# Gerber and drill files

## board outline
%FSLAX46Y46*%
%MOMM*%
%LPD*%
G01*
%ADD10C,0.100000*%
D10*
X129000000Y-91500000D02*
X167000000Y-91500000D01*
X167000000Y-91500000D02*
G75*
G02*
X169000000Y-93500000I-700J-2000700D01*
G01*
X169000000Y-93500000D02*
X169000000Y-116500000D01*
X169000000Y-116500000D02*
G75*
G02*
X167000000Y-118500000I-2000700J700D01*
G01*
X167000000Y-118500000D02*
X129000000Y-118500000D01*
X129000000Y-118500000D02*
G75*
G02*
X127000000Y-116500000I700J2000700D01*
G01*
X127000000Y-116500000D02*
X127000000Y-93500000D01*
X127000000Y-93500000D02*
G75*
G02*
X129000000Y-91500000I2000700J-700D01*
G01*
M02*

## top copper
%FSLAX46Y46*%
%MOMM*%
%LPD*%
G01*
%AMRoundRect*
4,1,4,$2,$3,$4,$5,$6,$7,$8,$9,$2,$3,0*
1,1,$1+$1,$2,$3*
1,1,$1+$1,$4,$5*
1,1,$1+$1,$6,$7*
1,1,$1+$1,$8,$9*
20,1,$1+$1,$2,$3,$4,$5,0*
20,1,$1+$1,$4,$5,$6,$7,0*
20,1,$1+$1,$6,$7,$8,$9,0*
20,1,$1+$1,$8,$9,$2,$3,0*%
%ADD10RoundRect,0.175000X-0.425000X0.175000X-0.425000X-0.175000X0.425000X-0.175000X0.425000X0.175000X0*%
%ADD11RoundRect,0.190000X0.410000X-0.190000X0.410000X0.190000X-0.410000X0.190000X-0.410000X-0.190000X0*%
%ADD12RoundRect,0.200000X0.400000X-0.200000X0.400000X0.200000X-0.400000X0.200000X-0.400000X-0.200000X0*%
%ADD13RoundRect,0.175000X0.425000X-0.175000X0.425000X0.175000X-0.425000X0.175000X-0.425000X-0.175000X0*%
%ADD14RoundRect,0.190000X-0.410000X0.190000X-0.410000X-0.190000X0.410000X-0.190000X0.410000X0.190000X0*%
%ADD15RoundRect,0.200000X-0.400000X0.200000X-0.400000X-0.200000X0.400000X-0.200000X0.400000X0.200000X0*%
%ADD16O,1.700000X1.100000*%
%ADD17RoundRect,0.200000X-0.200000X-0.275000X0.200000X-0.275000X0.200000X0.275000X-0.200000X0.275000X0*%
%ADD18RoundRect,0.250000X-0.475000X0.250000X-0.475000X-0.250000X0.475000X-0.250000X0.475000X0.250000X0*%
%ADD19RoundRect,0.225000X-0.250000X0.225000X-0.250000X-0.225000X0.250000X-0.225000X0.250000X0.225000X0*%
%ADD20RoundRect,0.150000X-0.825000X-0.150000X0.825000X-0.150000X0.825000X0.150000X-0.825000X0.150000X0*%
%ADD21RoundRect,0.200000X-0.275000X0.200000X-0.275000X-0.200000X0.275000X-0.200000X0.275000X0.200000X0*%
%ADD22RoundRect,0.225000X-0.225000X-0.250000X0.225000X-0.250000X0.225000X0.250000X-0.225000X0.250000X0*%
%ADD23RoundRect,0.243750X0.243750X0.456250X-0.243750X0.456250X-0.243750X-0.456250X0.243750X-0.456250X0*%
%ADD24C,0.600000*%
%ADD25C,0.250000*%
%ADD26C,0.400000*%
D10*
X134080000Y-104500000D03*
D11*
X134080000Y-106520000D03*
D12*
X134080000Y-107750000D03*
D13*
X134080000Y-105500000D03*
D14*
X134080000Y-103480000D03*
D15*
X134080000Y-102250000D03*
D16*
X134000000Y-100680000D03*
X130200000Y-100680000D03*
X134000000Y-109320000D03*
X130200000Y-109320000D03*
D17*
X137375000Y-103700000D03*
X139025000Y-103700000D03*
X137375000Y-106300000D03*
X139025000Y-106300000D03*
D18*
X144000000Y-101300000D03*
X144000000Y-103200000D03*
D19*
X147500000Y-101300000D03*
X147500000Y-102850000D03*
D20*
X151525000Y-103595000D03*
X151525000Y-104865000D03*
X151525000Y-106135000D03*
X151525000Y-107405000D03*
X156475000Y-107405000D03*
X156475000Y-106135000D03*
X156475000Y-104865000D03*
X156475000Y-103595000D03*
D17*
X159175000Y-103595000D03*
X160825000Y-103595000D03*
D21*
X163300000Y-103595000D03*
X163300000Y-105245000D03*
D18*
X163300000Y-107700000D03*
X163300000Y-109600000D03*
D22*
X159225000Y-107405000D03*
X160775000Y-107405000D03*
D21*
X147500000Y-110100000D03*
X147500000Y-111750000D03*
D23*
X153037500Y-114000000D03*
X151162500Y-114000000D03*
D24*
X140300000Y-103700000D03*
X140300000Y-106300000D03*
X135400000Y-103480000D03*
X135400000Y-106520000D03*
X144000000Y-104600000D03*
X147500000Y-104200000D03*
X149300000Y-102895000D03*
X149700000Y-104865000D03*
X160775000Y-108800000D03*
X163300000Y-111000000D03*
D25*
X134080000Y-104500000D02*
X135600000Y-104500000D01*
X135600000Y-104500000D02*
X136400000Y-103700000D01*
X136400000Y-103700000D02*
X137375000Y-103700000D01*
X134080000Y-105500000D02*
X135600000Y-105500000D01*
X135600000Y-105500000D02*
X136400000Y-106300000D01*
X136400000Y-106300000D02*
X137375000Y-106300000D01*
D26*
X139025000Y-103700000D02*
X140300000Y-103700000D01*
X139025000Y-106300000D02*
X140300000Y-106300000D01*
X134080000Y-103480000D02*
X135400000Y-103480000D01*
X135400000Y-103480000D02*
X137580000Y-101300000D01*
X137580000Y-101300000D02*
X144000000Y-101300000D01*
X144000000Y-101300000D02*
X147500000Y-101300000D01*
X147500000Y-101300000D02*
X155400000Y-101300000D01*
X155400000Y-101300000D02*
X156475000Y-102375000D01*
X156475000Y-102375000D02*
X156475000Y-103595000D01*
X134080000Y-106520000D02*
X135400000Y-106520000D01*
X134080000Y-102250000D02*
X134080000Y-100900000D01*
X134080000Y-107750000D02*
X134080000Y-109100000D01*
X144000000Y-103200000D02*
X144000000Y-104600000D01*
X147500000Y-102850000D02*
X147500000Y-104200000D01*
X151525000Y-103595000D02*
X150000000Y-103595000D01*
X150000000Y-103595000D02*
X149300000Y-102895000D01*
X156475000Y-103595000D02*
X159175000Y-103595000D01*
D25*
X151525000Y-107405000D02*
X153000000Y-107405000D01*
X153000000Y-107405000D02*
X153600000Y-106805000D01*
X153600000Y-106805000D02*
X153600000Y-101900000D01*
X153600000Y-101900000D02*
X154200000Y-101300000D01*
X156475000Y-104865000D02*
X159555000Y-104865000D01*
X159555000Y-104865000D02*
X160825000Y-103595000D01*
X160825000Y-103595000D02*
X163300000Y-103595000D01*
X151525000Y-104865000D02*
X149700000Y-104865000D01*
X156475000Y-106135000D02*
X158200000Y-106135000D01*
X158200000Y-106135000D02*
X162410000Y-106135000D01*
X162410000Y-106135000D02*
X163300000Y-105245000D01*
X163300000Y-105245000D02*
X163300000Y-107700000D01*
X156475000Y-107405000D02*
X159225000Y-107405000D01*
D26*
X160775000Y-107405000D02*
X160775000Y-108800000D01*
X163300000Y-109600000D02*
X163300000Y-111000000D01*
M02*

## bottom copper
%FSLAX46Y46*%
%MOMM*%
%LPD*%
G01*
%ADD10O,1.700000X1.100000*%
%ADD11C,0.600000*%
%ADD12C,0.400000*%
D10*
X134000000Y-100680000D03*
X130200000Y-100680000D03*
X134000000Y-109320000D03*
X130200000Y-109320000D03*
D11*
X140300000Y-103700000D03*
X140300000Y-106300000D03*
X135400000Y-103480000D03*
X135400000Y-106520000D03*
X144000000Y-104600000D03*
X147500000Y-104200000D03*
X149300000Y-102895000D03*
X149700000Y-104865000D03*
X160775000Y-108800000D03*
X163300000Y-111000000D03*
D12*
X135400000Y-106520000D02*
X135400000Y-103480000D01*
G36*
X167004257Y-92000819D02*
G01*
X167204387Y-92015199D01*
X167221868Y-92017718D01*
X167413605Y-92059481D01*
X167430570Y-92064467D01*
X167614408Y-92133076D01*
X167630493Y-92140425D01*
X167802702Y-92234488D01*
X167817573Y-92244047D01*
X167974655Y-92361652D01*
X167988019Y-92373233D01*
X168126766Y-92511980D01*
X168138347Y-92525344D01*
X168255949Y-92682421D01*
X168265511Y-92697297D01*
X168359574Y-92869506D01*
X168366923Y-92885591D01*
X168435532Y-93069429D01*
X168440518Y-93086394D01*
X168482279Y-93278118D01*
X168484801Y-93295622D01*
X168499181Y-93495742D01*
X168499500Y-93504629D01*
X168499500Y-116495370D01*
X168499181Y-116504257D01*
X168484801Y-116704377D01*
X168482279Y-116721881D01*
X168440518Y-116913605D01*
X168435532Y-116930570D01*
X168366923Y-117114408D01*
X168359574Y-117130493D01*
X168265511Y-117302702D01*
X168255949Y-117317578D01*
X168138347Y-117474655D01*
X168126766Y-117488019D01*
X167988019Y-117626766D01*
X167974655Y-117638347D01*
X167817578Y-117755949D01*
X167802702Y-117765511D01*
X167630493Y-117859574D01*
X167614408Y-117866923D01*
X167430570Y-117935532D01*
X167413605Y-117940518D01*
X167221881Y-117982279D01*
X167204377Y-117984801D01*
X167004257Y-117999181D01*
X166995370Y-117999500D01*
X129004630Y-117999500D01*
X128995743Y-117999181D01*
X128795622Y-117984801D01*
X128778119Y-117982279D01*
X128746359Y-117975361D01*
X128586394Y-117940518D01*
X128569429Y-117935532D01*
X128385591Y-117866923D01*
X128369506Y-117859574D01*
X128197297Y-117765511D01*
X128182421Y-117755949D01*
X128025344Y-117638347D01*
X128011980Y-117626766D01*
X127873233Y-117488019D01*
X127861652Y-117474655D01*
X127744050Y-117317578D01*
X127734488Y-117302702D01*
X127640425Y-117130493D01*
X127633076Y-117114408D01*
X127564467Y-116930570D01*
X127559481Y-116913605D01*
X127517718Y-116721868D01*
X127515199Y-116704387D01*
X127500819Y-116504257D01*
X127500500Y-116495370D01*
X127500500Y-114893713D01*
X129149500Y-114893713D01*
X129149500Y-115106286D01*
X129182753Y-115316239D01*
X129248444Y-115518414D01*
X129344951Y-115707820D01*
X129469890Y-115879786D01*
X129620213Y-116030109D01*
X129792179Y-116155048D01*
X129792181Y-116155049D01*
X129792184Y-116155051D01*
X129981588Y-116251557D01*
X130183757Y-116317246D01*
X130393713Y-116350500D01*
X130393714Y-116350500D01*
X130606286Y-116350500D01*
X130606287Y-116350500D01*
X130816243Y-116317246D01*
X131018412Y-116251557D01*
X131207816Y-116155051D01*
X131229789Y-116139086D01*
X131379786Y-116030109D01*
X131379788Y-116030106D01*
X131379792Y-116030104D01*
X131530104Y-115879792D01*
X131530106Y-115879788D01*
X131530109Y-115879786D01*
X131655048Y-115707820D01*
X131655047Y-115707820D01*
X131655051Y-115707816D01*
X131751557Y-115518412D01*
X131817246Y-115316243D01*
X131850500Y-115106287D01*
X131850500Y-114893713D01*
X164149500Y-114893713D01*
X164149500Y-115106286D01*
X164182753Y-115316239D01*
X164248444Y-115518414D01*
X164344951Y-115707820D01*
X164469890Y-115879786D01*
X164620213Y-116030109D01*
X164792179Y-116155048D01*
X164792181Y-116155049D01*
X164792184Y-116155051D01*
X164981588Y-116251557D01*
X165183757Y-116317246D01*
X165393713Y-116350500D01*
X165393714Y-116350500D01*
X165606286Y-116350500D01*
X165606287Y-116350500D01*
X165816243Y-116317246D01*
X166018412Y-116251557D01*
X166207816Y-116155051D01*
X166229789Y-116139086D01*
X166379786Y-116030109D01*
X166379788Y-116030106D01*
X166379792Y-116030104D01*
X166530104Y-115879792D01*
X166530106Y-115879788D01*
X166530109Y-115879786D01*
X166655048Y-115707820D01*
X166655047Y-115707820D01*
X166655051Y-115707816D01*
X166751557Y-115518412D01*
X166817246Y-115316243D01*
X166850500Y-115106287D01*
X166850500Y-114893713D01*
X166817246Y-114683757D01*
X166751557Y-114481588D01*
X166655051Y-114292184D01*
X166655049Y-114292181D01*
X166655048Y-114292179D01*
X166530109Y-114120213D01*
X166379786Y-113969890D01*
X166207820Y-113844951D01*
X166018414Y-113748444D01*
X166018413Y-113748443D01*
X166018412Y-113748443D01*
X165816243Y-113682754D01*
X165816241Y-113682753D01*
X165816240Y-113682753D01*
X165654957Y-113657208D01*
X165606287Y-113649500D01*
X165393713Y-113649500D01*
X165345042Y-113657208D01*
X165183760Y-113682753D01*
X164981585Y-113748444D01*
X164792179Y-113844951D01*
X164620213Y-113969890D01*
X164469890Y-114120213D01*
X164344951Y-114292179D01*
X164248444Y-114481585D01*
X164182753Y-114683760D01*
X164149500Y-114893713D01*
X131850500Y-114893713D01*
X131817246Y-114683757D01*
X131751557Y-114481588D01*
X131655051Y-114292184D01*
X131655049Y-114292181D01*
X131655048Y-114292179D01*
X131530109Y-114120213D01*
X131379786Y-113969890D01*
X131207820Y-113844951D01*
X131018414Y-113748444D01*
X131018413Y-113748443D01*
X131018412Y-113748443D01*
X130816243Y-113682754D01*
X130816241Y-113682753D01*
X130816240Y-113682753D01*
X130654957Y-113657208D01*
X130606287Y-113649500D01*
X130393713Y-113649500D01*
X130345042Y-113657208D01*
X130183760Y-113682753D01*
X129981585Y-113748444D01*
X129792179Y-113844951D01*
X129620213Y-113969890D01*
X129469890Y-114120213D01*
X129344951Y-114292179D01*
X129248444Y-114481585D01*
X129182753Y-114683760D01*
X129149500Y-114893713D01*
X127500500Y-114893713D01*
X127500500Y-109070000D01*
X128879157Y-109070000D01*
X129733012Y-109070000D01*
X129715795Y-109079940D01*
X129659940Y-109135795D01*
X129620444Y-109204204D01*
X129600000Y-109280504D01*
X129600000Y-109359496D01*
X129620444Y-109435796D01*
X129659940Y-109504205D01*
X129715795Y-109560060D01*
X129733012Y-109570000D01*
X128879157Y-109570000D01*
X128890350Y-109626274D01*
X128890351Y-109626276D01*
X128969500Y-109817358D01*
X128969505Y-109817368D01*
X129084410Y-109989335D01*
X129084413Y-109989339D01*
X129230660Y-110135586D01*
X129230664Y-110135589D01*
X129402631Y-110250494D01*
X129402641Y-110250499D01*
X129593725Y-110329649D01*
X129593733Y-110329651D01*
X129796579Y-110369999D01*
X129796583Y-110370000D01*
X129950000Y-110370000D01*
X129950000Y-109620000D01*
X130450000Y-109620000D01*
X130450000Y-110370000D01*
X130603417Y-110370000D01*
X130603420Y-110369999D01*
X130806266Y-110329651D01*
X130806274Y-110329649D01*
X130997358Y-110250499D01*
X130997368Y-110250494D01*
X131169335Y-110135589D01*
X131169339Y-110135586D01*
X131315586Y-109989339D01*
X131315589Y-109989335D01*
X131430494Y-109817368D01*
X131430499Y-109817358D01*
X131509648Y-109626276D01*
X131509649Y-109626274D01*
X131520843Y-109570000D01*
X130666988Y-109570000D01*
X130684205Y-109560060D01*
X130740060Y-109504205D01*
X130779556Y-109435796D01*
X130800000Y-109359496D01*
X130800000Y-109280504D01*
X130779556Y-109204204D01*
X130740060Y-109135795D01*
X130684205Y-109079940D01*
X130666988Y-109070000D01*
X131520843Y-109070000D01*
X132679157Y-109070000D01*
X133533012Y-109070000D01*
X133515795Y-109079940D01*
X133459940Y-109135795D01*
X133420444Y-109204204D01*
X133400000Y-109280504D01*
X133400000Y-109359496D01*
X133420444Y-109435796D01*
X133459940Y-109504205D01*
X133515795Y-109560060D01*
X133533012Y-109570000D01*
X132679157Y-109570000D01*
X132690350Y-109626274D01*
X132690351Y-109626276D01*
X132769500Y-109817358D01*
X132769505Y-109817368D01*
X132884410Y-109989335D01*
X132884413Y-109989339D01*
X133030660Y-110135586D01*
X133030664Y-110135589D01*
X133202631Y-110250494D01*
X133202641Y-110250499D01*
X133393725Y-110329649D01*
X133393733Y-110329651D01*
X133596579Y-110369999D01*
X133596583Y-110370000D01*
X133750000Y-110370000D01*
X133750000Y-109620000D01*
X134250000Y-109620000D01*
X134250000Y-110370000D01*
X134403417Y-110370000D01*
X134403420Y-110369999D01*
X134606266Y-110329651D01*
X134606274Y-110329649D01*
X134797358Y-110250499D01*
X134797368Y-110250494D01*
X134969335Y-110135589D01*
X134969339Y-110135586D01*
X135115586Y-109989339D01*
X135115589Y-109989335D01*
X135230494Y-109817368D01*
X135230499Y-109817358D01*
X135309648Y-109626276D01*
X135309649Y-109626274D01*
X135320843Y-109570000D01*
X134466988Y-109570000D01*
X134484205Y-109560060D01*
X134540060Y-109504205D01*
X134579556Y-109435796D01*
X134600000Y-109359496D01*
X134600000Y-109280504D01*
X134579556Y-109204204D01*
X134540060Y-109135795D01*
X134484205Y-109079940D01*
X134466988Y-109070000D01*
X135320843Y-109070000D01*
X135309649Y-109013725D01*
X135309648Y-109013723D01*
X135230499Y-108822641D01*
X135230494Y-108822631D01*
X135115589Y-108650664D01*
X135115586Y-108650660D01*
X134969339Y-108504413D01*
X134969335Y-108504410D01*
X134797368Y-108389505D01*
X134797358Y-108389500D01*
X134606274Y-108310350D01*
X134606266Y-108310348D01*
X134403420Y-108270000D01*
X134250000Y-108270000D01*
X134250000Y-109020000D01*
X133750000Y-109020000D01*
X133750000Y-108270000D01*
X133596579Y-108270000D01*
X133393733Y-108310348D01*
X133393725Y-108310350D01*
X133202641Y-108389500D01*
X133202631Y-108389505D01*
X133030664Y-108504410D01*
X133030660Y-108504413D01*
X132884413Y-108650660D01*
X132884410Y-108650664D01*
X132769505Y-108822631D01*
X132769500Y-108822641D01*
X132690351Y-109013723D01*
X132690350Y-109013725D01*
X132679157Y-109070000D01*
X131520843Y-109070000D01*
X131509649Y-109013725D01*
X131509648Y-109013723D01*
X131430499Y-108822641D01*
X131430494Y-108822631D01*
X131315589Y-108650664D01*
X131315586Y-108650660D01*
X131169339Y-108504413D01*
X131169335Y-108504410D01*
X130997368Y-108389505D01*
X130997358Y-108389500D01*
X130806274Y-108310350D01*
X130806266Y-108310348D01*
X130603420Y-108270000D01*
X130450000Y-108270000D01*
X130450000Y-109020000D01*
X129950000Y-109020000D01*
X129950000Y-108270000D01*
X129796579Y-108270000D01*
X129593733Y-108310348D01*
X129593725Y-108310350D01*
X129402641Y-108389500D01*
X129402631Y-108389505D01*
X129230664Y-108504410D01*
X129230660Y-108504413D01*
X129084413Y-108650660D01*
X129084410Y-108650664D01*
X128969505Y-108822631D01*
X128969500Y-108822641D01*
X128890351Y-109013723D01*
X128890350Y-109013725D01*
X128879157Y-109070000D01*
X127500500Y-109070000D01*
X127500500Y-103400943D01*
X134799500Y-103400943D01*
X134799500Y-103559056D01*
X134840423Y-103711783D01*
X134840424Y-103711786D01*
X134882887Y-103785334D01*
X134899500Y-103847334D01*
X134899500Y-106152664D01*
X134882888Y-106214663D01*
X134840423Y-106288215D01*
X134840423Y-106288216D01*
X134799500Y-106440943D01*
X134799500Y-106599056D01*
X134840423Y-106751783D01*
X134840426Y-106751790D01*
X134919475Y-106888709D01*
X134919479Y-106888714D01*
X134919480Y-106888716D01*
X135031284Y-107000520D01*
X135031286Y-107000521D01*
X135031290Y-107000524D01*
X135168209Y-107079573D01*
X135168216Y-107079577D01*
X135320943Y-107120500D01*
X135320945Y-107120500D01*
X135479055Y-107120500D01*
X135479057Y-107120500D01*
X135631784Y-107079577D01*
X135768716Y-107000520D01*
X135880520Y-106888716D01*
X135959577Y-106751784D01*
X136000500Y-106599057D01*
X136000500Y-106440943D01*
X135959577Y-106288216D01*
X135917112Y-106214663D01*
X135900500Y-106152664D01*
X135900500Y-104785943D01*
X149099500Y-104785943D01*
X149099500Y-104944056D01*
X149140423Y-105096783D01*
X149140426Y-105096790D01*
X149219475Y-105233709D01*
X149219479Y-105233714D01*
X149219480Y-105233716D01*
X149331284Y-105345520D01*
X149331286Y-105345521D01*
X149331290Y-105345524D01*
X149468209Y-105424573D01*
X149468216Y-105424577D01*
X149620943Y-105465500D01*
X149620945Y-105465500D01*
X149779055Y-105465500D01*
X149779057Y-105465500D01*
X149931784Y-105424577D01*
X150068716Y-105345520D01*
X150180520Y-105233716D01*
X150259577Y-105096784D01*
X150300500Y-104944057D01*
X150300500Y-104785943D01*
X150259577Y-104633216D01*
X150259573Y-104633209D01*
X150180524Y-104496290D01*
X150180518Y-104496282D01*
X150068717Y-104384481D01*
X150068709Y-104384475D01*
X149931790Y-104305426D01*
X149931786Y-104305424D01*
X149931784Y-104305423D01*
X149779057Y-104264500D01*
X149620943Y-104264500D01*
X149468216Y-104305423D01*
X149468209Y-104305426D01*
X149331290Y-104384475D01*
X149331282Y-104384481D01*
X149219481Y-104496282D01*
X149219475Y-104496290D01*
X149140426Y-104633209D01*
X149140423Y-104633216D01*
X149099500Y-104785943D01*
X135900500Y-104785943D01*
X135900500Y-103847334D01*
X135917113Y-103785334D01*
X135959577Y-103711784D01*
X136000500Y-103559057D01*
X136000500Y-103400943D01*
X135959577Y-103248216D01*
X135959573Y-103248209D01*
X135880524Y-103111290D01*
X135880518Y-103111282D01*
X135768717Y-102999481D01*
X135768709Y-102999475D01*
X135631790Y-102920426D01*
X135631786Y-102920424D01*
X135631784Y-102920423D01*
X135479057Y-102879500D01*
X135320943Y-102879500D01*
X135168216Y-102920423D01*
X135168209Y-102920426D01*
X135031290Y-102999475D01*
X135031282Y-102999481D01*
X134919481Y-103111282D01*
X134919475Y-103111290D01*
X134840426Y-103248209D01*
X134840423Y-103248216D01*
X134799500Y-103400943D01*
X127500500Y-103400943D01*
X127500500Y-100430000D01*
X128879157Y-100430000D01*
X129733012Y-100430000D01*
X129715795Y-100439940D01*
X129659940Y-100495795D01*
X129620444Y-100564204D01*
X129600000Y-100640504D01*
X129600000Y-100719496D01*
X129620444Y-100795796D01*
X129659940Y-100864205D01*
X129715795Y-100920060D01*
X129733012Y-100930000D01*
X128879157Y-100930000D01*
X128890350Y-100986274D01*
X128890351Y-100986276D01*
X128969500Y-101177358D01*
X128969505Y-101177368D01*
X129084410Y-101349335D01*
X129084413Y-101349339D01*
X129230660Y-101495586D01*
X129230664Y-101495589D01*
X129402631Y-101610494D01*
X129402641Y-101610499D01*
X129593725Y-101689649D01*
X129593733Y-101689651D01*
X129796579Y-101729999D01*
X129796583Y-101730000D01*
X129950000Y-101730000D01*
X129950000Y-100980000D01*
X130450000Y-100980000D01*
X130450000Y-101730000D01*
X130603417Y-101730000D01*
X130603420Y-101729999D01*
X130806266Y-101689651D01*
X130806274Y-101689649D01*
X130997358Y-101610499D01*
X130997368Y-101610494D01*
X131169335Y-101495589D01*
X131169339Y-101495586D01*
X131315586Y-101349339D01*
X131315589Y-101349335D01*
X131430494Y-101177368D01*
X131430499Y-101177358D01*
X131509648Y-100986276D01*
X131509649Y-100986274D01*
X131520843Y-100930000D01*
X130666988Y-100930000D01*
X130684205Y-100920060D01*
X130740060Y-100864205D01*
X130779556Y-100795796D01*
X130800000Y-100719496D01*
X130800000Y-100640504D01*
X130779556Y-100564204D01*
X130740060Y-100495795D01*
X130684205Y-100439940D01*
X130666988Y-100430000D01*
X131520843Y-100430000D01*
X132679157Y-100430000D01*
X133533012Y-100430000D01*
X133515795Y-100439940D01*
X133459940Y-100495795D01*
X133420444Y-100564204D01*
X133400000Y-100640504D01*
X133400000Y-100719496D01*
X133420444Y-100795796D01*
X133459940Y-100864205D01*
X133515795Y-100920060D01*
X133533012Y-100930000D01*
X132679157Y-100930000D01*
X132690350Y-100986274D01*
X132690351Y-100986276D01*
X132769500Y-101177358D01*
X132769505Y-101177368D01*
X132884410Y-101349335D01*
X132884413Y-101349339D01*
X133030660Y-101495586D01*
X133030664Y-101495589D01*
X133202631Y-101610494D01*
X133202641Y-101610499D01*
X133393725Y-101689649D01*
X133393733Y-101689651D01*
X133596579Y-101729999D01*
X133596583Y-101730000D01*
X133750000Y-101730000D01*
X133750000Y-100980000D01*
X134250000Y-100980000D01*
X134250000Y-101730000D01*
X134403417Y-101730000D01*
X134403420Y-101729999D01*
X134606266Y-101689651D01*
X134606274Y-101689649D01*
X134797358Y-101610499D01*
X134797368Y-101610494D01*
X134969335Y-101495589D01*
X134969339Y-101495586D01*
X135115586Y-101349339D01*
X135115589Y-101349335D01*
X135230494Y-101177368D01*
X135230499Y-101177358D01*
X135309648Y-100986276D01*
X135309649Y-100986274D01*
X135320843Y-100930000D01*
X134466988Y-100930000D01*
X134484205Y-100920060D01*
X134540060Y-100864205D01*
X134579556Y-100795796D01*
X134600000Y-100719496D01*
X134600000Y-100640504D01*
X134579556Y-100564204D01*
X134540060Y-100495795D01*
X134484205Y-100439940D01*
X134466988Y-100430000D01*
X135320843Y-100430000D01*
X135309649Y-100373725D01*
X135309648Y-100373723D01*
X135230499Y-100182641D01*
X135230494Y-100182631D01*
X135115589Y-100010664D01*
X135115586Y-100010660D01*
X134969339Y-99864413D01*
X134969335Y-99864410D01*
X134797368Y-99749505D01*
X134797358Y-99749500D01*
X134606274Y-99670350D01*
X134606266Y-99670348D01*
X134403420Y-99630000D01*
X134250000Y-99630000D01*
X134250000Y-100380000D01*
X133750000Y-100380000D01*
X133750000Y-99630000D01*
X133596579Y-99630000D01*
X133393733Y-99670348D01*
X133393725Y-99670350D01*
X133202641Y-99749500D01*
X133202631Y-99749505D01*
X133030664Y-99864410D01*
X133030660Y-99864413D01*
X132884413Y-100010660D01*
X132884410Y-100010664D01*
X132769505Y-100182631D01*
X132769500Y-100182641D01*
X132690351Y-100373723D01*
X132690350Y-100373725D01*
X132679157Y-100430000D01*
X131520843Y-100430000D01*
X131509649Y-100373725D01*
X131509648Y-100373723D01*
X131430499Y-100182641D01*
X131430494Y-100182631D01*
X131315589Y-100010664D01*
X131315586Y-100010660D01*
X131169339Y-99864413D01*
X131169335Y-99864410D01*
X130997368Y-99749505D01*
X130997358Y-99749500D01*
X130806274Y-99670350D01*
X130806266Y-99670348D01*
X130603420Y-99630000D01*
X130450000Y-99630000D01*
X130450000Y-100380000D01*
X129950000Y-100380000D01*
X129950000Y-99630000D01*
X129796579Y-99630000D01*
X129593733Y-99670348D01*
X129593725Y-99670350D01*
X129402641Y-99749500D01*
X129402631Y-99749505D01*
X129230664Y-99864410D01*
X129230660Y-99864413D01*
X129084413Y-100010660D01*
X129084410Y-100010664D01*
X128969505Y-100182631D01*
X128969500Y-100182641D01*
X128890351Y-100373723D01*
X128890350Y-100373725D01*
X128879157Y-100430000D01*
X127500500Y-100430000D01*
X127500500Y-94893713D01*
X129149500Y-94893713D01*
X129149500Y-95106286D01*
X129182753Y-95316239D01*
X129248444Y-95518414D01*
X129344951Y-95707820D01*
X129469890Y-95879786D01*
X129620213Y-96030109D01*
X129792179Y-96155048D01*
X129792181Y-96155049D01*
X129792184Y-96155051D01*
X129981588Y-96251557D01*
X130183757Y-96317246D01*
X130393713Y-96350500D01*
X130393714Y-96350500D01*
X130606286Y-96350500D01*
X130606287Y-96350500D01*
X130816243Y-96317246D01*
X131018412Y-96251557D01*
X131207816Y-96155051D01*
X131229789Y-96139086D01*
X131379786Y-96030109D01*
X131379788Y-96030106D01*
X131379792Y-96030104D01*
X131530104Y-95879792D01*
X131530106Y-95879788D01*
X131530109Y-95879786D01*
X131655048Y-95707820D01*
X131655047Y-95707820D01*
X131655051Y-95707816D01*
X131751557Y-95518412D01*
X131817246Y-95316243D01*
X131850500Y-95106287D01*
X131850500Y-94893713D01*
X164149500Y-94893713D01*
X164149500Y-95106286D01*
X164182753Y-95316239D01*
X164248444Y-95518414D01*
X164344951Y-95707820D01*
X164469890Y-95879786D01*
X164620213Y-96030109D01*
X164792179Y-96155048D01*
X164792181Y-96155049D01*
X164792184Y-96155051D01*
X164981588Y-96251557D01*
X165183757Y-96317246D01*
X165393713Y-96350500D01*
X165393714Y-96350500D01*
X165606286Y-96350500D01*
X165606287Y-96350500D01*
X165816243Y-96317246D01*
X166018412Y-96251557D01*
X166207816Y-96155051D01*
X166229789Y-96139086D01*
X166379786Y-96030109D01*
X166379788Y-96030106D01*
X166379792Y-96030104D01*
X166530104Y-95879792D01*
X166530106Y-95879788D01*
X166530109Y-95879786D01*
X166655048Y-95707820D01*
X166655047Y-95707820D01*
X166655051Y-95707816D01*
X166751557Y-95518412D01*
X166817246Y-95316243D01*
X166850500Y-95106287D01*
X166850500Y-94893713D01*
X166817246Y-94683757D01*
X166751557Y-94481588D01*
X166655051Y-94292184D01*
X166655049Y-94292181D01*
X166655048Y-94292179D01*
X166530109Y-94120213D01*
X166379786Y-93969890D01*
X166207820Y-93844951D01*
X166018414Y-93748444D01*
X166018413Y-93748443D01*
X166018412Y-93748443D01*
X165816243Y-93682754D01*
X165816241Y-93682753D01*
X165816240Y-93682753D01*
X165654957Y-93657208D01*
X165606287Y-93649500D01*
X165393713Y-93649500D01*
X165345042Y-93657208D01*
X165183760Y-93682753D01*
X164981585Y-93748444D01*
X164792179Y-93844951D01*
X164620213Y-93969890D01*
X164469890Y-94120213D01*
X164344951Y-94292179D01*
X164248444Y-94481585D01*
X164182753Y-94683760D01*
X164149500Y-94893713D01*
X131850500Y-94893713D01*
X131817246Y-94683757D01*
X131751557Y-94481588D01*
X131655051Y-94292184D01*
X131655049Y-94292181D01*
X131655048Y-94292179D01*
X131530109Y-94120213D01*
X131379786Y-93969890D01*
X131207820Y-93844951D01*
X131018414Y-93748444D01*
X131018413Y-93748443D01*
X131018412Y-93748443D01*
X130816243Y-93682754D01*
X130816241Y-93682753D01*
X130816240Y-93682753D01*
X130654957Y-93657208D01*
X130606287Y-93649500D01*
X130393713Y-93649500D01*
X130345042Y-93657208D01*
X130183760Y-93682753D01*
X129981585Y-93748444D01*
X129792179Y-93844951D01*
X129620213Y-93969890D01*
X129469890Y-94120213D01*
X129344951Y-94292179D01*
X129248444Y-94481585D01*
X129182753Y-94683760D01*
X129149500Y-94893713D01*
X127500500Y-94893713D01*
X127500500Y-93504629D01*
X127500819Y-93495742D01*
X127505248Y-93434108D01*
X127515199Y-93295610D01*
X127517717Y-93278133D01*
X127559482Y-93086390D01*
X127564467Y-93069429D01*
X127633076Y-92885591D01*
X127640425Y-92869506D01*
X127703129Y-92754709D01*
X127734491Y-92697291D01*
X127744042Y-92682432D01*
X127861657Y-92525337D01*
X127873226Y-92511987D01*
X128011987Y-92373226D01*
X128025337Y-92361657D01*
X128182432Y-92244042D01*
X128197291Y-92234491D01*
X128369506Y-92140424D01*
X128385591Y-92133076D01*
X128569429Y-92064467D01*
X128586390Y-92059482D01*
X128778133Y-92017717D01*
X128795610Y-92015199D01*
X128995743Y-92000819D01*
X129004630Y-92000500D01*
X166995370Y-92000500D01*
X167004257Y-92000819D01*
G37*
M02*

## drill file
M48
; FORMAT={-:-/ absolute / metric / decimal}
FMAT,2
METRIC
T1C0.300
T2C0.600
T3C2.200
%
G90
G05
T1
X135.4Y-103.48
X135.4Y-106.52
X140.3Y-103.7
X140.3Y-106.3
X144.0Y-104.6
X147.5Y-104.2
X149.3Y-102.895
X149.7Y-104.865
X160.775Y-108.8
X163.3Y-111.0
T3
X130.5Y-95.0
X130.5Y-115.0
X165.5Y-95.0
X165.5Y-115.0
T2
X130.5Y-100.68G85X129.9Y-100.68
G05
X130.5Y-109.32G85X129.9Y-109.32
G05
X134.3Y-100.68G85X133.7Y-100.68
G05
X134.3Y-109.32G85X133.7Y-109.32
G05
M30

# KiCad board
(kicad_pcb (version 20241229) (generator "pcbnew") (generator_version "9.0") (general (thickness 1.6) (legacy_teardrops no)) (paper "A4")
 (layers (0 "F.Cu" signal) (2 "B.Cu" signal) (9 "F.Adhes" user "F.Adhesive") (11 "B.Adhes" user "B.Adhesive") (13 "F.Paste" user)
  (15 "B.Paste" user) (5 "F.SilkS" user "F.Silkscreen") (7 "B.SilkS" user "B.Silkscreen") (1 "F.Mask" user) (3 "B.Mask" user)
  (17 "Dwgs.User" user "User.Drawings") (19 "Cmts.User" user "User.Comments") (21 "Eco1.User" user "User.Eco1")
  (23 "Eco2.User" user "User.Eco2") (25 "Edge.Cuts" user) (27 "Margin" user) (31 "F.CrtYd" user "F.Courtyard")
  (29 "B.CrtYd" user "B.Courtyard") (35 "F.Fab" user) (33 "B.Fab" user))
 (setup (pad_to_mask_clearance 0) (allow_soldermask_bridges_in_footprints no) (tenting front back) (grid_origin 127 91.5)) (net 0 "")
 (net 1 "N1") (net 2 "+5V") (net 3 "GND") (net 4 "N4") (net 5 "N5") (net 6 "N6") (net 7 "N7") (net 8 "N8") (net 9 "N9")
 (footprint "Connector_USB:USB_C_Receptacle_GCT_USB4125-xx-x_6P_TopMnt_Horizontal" (layer "F.Cu") (at 131 105 270)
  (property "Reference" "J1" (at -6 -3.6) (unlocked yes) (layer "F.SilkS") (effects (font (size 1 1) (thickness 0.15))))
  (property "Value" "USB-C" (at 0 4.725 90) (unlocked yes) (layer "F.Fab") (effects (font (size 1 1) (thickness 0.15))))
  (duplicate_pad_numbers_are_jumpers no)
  (pad "A5" smd roundrect (at -0.5 -3.08 270) (size 0.7 1.2) (layers "F.Cu" "F.Mask" "F.Paste") (roundrect_rratio 0.25) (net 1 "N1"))
  (pad "A9" smd roundrect (at 1.52 -3.08 90) (size 0.76 1.2) (layers "F.Cu" "F.Mask" "F.Paste") (roundrect_rratio 0.25) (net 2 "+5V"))
  (pad "A12" smd roundrect (at 2.75 -3.08 90) (size 0.8 1.2) (layers "F.Cu" "F.Mask" "F.Paste") (roundrect_rratio 0.25) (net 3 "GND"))
  (pad "B5" smd roundrect (at 0.5 -3.08 90) (size 0.7 1.2) (layers "F.Cu" "F.Mask" "F.Paste") (roundrect_rratio 0.25) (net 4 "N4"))
  (pad "B9" smd roundrect (at -1.52 -3.08 270) (size 0.76 1.2) (layers "F.Cu" "F.Mask" "F.Paste") (roundrect_rratio 0.25) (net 2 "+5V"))
  (pad "B12" smd roundrect (at -2.75 -3.08 270) (size 0.8 1.2) (layers "F.Cu" "F.Mask" "F.Paste") (roundrect_rratio 0.25) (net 3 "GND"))
  (pad "SH" thru_hole oval (at -4.32 -3 270) (size 1.1 1.7) (drill oval 0.6 1.2) (layers "*.Cu" "*.Mask" "F.Paste")
   (remove_unused_layers no) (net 3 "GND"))
  (pad "SH" thru_hole oval (at -4.32 0.8 270) (size 1.1 1.7) (drill oval 0.6 1.2) (layers "*.Cu" "*.Mask" "F.Paste")
   (remove_unused_layers no) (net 3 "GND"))
  (pad "SH" thru_hole oval (at 4.32 -3 270) (size 1.1 1.7) (drill oval 0.6 1.2) (layers "*.Cu" "*.Mask" "F.Paste") (remove_unused_layers no)
   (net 3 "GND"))
  (pad "SH" thru_hole oval (at 4.32 0.8 270) (size 1.1 1.7) (drill oval 0.6 1.2) (layers "*.Cu" "*.Mask" "F.Paste")
   (remove_unused_layers no) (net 3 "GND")))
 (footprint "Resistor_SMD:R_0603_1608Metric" (layer "F.Cu") (at 138.2 103.7)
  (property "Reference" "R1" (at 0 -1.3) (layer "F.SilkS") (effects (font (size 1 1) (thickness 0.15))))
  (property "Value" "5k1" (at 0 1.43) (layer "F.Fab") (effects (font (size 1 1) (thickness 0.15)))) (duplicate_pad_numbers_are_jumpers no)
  (pad "1" smd roundrect (at -0.825 0) (size 0.8 0.95) (layers "F.Cu" "F.Mask" "F.Paste") (roundrect_rratio 0.25) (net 1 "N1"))
  (pad "2" smd roundrect (at 0.825 0) (size 0.8 0.95) (layers "F.Cu" "F.Mask" "F.Paste") (roundrect_rratio 0.25) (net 3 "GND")))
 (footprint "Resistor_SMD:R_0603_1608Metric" (layer "F.Cu") (at 138.2 106.3)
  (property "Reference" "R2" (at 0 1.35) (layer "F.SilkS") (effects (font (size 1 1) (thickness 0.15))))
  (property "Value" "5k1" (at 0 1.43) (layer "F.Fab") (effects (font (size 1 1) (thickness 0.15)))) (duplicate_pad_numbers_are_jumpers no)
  (pad "1" smd roundrect (at -0.825 0) (size 0.8 0.95) (layers "F.Cu" "F.Mask" "F.Paste") (roundrect_rratio 0.25) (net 4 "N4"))
  (pad "2" smd roundrect (at 0.825 0) (size 0.8 0.95) (layers "F.Cu" "F.Mask" "F.Paste") (roundrect_rratio 0.25) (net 3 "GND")))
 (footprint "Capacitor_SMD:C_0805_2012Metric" (layer "F.Cu") (at 144 102.25 270)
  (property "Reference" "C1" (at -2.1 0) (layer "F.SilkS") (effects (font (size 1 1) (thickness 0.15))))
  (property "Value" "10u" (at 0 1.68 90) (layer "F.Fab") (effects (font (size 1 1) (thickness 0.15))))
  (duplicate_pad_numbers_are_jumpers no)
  (pad "1" smd roundrect (at -0.95 0 270) (size 1 1.45) (layers "F.Cu" "F.Mask" "F.Paste") (roundrect_rratio 0.25) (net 2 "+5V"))
  (pad "2" smd roundrect (at 0.95 0 270) (size 1 1.45) (layers "F.Cu" "F.Mask" "F.Paste") (roundrect_rratio 0.25) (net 3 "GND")))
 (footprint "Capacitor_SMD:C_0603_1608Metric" (layer "F.Cu") (at 147.5 102.075 270)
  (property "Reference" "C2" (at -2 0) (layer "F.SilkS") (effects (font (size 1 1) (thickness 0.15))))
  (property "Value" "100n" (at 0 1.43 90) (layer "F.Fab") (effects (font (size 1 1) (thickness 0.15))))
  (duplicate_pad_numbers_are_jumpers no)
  (pad "1" smd roundrect (at -0.775 0 270) (size 0.9 0.95) (layers "F.Cu" "F.Mask" "F.Paste") (roundrect_rratio 0.25) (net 2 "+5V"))
  (pad "2" smd roundrect (at 0.775 0 270) (size 0.9 0.95) (layers "F.Cu" "F.Mask" "F.Paste") (roundrect_rratio 0.25) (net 3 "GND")))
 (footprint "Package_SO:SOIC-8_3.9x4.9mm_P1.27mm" (layer "F.Cu") (at 154 105.5)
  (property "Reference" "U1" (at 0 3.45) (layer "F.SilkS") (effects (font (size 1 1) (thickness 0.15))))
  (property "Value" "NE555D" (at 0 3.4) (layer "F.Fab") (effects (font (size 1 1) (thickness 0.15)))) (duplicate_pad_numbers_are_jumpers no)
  (pad "1" smd roundrect (at -2.475 -1.905) (size 1.95 0.6) (layers "F.Cu" "F.Mask" "F.Paste") (roundrect_rratio 0.25) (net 3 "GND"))
  (pad "2" smd roundrect (at -2.475 -0.635) (size 1.95 0.6) (layers "F.Cu" "F.Mask" "F.Paste") (roundrect_rratio 0.25) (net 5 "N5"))
  (pad "3" smd roundrect (at -2.475 0.635) (size 1.95 0.6) (layers "F.Cu" "F.Mask" "F.Paste") (roundrect_rratio 0.25) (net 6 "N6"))
  (pad "4" smd roundrect (at -2.475 1.905) (size 1.95 0.6) (layers "F.Cu" "F.Mask" "F.Paste") (roundrect_rratio 0.25) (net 2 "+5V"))
  (pad "5" smd roundrect (at 2.475 1.905) (size 1.95 0.6) (layers "F.Cu" "F.Mask" "F.Paste") (roundrect_rratio 0.25) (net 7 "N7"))
  (pad "6" smd roundrect (at 2.475 0.635) (size 1.95 0.6) (layers "F.Cu" "F.Mask" "F.Paste") (roundrect_rratio 0.25) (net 5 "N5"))
  (pad "7" smd roundrect (at 2.475 -0.635) (size 1.95 0.6) (layers "F.Cu" "F.Mask" "F.Paste") (roundrect_rratio 0.25) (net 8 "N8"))
  (pad "8" smd roundrect (at 2.475 -1.905) (size 1.95 0.6) (layers "F.Cu" "F.Mask" "F.Paste") (roundrect_rratio 0.25) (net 2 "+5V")))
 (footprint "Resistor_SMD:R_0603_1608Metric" (layer "F.Cu") (at 160 103.595)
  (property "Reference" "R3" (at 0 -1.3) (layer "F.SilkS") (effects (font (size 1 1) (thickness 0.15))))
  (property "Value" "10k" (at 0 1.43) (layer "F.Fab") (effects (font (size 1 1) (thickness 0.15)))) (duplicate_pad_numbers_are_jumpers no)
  (pad "1" smd roundrect (at -0.825 0) (size 0.8 0.95) (layers "F.Cu" "F.Mask" "F.Paste") (roundrect_rratio 0.25) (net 2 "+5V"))
  (pad "2" smd roundrect (at 0.825 0) (size 0.8 0.95) (layers "F.Cu" "F.Mask" "F.Paste") (roundrect_rratio 0.25) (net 8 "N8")))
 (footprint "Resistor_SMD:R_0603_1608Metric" (layer "F.Cu") (at 163.3 104.42 270)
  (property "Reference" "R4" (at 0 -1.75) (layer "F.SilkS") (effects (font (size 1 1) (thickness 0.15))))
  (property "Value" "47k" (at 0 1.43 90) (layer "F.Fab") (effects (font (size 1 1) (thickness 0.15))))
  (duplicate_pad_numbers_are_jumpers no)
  (pad "1" smd roundrect (at -0.825 0 270) (size 0.8 0.95) (layers "F.Cu" "F.Mask" "F.Paste") (roundrect_rratio 0.25) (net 8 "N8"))
  (pad "2" smd roundrect (at 0.825 0 270) (size 0.8 0.95) (layers "F.Cu" "F.Mask" "F.Paste") (roundrect_rratio 0.25) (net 5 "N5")))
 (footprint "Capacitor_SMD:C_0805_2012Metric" (layer "F.Cu") (at 163.3 108.65 270)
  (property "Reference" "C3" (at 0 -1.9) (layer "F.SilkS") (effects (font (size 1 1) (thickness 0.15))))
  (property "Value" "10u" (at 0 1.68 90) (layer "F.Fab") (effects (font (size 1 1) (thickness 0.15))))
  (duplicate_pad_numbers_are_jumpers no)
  (pad "1" smd roundrect (at -0.95 0 270) (size 1 1.45) (layers "F.Cu" "F.Mask" "F.Paste") (roundrect_rratio 0.25) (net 5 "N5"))
  (pad "2" smd roundrect (at 0.95 0 270) (size 1 1.45) (layers "F.Cu" "F.Mask" "F.Paste") (roundrect_rratio 0.25) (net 3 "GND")))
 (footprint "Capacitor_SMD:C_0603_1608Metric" (layer "F.Cu") (at 160 107.405)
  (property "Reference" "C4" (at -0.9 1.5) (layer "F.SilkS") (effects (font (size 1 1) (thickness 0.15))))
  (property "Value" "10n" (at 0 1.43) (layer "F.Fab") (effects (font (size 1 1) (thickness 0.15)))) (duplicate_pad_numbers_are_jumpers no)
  (pad "1" smd roundrect (at -0.775 0) (size 0.9 0.95) (layers "F.Cu" "F.Mask" "F.Paste") (roundrect_rratio 0.25) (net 7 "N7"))
  (pad "2" smd roundrect (at 0.775 0) (size 0.9 0.95) (layers "F.Cu" "F.Mask" "F.Paste") (roundrect_rratio 0.25) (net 3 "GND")))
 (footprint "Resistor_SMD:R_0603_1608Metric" (layer "F.Cu") (at 147.5 110.925 270)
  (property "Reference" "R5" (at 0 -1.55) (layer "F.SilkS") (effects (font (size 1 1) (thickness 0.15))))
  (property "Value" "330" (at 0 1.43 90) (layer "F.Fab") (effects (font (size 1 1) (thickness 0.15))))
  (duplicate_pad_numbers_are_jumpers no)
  (pad "1" smd roundrect (at -0.825 0 270) (size 0.8 0.95) (layers "F.Cu" "F.Mask" "F.Paste") (roundrect_rratio 0.25) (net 6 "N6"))
  (pad "2" smd roundrect (at 0.825 0 270) (size 0.8 0.95) (layers "F.Cu" "F.Mask" "F.Paste") (roundrect_rratio 0.25) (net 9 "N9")))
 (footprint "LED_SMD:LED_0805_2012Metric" (layer "F.Cu") (at 152.1 114 180)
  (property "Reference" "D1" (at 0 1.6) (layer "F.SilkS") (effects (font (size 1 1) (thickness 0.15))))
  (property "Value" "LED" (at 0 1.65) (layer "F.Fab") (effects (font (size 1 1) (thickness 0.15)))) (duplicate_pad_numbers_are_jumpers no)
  (pad "1" smd roundrect (at -0.9375 0 180) (size 0.975 1.4) (layers "F.Cu" "F.Mask" "F.Paste") (roundrect_rratio 0.25) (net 3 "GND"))
  (pad "2" smd roundrect (at 0.9375 0 180) (size 0.975 1.4) (layers "F.Cu" "F.Mask" "F.Paste") (roundrect_rratio 0.25) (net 9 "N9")))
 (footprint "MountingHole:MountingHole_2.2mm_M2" (layer "F.Cu") (at 130.5 95)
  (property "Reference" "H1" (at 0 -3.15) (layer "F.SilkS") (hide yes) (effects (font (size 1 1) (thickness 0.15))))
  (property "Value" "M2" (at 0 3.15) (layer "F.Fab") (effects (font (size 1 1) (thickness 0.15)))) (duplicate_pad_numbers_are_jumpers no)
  (pad "" np_thru_hole circle (at 0 0) (size 2.2 2.2) (drill 2.2) (layers "*.Cu" "*.Mask")))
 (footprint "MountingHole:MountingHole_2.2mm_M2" (layer "F.Cu") (at 165.5 95)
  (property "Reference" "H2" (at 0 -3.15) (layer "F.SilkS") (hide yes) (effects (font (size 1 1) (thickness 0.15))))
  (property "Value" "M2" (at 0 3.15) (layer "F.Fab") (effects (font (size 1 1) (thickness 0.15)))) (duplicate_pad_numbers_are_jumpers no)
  (pad "" np_thru_hole circle (at 0 0) (size 2.2 2.2) (drill 2.2) (layers "*.Cu" "*.Mask")))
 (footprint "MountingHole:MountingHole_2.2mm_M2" (layer "F.Cu") (at 130.5 115)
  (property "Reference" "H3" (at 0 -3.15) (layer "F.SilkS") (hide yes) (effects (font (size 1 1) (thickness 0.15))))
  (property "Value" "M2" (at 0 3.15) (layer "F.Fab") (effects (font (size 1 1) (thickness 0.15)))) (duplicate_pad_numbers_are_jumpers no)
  (pad "" np_thru_hole circle (at 0 0) (size 2.2 2.2) (drill 2.2) (layers "*.Cu" "*.Mask")))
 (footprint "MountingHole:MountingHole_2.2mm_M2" (layer "F.Cu") (at 165.5 115)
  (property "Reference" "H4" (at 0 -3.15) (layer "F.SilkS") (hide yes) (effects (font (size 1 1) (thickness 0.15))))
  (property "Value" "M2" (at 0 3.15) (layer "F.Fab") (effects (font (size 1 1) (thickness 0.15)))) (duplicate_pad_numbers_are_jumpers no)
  (pad "" np_thru_hole circle (at 0 0) (size 2.2 2.2) (drill 2.2) (layers "*.Cu" "*.Mask")))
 (segment (start 134.08 104.5) (end 135.6 104.5) (width 0.25) (layer "F.Cu") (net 1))
 (segment (start 135.6 104.5) (end 136.4 103.7) (width 0.25) (layer "F.Cu") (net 1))
 (segment (start 136.4 103.7) (end 137.375 103.7) (width 0.25) (layer "F.Cu") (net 1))
 (segment (start 134.08 105.5) (end 135.6 105.5) (width 0.25) (layer "F.Cu") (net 4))
 (segment (start 135.6 105.5) (end 136.4 106.3) (width 0.25) (layer "F.Cu") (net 4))
 (segment (start 136.4 106.3) (end 137.375 106.3) (width 0.25) (layer "F.Cu") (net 4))
 (segment (start 139.025 103.7) (end 140.3 103.7) (width 0.4) (layer "F.Cu") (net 3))
 (via (at 140.3 103.7) (size 0.6) (drill 0.3) (layers "F.Cu" "B.Cu") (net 3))
 (segment (start 139.025 106.3) (end 140.3 106.3) (width 0.4) (layer "F.Cu") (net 3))
 (via (at 140.3 106.3) (size 0.6) (drill 0.3) (layers "F.Cu" "B.Cu") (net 3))
 (segment (start 134.08 103.48) (end 135.4 103.48) (width 0.4) (layer "F.Cu") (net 2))
 (via (at 135.4 103.48) (size 0.6) (drill 0.3) (layers "F.Cu" "B.Cu") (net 2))
 (segment (start 135.4 103.48) (end 137.58 101.3) (width 0.4) (layer "F.Cu") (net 2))
 (segment (start 137.58 101.3) (end 144 101.3) (width 0.4) (layer "F.Cu") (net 2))
 (segment (start 144 101.3) (end 147.5 101.3) (width 0.4) (layer "F.Cu") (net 2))
 (segment (start 147.5 101.3) (end 155.4 101.3) (width 0.4) (layer "F.Cu") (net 2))
 (segment (start 155.4 101.3) (end 156.475 102.375) (width 0.4) (layer "F.Cu") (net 2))
 (segment (start 156.475 102.375) (end 156.475 103.595) (width 0.4) (layer "F.Cu") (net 2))
 (segment (start 134.08 106.52) (end 135.4 106.52) (width 0.4) (layer "F.Cu") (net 2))
 (via (at 135.4 106.52) (size 0.6) (drill 0.3) (layers "F.Cu" "B.Cu") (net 2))
 (segment (start 135.4 106.52) (end 135.4 103.48) (width 0.4) (layer "B.Cu") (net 2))
 (segment (start 134.08 102.25) (end 134.08 100.9) (width 0.4) (layer "F.Cu") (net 3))
 (segment (start 134.08 107.75) (end 134.08 109.1) (width 0.4) (layer "F.Cu") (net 3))
 (segment (start 144 103.2) (end 144 104.6) (width 0.4) (layer "F.Cu") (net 3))
 (via (at 144 104.6) (size 0.6) (drill 0.3) (layers "F.Cu" "B.Cu") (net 3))
 (segment (start 147.5 102.85) (end 147.5 104.2) (width 0.4) (layer "F.Cu") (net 3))
 (via (at 147.5 104.2) (size 0.6) (drill 0.3) (layers "F.Cu" "B.Cu") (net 3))
 (segment (start 151.525 103.595) (end 150 103.595) (width 0.4) (layer "F.Cu") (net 3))
 (segment (start 150 103.595) (end 149.3 102.895) (width 0.4) (layer "F.Cu") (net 3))
 (via (at 149.3 102.895) (size 0.6) (drill 0.3) (layers "F.Cu" "B.Cu") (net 3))
 (segment (start 156.475 103.595) (end 159.175 103.595) (width 0.4) (layer "F.Cu") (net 2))
 (segment (start 151.525 107.405) (end 153 107.405) (width 0.25) (layer "F.Cu") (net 2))
 (segment (start 153 107.405) (end 153.6 106.805) (width 0.25) (layer "F.Cu") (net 2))
 (segment (start 153.6 106.805) (end 153.6 101.9) (width 0.25) (layer "F.Cu") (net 2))
 (segment (start 153.6 101.9) (end 154.2 101.3) (width 0.25) (layer "F.Cu") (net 2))
 (segment (start 156.475 104.865) (end 159.555 104.865) (width 0.25) (layer "F.Cu") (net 8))
 (segment (start 159.555 104.865) (end 160.825 103.595) (width 0.25) (layer "F.Cu") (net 8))
 (segment (start 160.825 103.595) (end 163.3 103.595) (width 0.25) (layer "F.Cu") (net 8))
 (segment (start 151.525 104.865) (end 149.7 104.865) (width 0.25) (layer "F.Cu") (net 5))
 (via (at 149.7 104.865) (size 0.6) (drill 0.3) (layers "F.Cu" "B.Cu") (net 5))
 (segment (start 156.475 106.135) (end 158.2 106.135) (width 0.25) (layer "F.Cu") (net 5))
 (segment (start 158.2 106.135) (end 162.41 106.135) (width 0.25) (layer "F.Cu") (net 5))
 (segment (start 162.41 106.135) (end 163.3 105.245) (width 0.25) (layer "F.Cu") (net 5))
 (segment (start 163.3 105.245) (end 163.3 107.7) (width 0.25) (layer "F.Cu") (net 5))
 (segment (start 156.475 107.405) (end 159.225 107.405) (width 0.25) (layer "F.Cu") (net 7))
 (segment (start 160.775 107.405) (end 160.775 108.8) (width 0.4) (layer "F.Cu") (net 3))
 (via (at 160.775 108.8) (size 0.6) (drill 0.3) (layers "F.Cu" "B.Cu") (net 3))
 (segment (start 163.3 109.6) (end 163.3 111) (width 0.4) (layer "F.Cu") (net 3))
 (via (at 163.3 111) (size 0.6) (drill 0.3) (layers "F.Cu" "B.Cu") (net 3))
 (gr_line (start 129 91.5) (end 167 91.5) (stroke (width 0.1) (type default)) (layer "Edge.Cuts"))
 (gr_arc (start 167 91.5) (mid 168.414 92.086) (end 169 93.5) (stroke (width 0.1) (type default)) (layer "Edge.Cuts"))
 (gr_line (start 169 93.5) (end 169 116.5) (stroke (width 0.1) (type default)) (layer "Edge.Cuts"))
 (gr_arc (start 169 116.5) (mid 168.414 117.914) (end 167 118.5) (stroke (width 0.1) (type default)) (layer "Edge.Cuts"))
 (gr_line (start 167 118.5) (end 129 118.5) (stroke (width 0.1) (type default)) (layer "Edge.Cuts"))
 (gr_arc (start 129 118.5) (mid 127.586 117.914) (end 127 116.5) (stroke (width 0.1) (type default)) (layer "Edge.Cuts"))
 (gr_line (start 127 116.5) (end 127 93.5) (stroke (width 0.1) (type default)) (layer "Edge.Cuts"))
 (gr_arc (start 127 93.5) (mid 127.586 92.086) (end 129 91.5) (stroke (width 0.1) (type default)) (layer "Edge.Cuts"))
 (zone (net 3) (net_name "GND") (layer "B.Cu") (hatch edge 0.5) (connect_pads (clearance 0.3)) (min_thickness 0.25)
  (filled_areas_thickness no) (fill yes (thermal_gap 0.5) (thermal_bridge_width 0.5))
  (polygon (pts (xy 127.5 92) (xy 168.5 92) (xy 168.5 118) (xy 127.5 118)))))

